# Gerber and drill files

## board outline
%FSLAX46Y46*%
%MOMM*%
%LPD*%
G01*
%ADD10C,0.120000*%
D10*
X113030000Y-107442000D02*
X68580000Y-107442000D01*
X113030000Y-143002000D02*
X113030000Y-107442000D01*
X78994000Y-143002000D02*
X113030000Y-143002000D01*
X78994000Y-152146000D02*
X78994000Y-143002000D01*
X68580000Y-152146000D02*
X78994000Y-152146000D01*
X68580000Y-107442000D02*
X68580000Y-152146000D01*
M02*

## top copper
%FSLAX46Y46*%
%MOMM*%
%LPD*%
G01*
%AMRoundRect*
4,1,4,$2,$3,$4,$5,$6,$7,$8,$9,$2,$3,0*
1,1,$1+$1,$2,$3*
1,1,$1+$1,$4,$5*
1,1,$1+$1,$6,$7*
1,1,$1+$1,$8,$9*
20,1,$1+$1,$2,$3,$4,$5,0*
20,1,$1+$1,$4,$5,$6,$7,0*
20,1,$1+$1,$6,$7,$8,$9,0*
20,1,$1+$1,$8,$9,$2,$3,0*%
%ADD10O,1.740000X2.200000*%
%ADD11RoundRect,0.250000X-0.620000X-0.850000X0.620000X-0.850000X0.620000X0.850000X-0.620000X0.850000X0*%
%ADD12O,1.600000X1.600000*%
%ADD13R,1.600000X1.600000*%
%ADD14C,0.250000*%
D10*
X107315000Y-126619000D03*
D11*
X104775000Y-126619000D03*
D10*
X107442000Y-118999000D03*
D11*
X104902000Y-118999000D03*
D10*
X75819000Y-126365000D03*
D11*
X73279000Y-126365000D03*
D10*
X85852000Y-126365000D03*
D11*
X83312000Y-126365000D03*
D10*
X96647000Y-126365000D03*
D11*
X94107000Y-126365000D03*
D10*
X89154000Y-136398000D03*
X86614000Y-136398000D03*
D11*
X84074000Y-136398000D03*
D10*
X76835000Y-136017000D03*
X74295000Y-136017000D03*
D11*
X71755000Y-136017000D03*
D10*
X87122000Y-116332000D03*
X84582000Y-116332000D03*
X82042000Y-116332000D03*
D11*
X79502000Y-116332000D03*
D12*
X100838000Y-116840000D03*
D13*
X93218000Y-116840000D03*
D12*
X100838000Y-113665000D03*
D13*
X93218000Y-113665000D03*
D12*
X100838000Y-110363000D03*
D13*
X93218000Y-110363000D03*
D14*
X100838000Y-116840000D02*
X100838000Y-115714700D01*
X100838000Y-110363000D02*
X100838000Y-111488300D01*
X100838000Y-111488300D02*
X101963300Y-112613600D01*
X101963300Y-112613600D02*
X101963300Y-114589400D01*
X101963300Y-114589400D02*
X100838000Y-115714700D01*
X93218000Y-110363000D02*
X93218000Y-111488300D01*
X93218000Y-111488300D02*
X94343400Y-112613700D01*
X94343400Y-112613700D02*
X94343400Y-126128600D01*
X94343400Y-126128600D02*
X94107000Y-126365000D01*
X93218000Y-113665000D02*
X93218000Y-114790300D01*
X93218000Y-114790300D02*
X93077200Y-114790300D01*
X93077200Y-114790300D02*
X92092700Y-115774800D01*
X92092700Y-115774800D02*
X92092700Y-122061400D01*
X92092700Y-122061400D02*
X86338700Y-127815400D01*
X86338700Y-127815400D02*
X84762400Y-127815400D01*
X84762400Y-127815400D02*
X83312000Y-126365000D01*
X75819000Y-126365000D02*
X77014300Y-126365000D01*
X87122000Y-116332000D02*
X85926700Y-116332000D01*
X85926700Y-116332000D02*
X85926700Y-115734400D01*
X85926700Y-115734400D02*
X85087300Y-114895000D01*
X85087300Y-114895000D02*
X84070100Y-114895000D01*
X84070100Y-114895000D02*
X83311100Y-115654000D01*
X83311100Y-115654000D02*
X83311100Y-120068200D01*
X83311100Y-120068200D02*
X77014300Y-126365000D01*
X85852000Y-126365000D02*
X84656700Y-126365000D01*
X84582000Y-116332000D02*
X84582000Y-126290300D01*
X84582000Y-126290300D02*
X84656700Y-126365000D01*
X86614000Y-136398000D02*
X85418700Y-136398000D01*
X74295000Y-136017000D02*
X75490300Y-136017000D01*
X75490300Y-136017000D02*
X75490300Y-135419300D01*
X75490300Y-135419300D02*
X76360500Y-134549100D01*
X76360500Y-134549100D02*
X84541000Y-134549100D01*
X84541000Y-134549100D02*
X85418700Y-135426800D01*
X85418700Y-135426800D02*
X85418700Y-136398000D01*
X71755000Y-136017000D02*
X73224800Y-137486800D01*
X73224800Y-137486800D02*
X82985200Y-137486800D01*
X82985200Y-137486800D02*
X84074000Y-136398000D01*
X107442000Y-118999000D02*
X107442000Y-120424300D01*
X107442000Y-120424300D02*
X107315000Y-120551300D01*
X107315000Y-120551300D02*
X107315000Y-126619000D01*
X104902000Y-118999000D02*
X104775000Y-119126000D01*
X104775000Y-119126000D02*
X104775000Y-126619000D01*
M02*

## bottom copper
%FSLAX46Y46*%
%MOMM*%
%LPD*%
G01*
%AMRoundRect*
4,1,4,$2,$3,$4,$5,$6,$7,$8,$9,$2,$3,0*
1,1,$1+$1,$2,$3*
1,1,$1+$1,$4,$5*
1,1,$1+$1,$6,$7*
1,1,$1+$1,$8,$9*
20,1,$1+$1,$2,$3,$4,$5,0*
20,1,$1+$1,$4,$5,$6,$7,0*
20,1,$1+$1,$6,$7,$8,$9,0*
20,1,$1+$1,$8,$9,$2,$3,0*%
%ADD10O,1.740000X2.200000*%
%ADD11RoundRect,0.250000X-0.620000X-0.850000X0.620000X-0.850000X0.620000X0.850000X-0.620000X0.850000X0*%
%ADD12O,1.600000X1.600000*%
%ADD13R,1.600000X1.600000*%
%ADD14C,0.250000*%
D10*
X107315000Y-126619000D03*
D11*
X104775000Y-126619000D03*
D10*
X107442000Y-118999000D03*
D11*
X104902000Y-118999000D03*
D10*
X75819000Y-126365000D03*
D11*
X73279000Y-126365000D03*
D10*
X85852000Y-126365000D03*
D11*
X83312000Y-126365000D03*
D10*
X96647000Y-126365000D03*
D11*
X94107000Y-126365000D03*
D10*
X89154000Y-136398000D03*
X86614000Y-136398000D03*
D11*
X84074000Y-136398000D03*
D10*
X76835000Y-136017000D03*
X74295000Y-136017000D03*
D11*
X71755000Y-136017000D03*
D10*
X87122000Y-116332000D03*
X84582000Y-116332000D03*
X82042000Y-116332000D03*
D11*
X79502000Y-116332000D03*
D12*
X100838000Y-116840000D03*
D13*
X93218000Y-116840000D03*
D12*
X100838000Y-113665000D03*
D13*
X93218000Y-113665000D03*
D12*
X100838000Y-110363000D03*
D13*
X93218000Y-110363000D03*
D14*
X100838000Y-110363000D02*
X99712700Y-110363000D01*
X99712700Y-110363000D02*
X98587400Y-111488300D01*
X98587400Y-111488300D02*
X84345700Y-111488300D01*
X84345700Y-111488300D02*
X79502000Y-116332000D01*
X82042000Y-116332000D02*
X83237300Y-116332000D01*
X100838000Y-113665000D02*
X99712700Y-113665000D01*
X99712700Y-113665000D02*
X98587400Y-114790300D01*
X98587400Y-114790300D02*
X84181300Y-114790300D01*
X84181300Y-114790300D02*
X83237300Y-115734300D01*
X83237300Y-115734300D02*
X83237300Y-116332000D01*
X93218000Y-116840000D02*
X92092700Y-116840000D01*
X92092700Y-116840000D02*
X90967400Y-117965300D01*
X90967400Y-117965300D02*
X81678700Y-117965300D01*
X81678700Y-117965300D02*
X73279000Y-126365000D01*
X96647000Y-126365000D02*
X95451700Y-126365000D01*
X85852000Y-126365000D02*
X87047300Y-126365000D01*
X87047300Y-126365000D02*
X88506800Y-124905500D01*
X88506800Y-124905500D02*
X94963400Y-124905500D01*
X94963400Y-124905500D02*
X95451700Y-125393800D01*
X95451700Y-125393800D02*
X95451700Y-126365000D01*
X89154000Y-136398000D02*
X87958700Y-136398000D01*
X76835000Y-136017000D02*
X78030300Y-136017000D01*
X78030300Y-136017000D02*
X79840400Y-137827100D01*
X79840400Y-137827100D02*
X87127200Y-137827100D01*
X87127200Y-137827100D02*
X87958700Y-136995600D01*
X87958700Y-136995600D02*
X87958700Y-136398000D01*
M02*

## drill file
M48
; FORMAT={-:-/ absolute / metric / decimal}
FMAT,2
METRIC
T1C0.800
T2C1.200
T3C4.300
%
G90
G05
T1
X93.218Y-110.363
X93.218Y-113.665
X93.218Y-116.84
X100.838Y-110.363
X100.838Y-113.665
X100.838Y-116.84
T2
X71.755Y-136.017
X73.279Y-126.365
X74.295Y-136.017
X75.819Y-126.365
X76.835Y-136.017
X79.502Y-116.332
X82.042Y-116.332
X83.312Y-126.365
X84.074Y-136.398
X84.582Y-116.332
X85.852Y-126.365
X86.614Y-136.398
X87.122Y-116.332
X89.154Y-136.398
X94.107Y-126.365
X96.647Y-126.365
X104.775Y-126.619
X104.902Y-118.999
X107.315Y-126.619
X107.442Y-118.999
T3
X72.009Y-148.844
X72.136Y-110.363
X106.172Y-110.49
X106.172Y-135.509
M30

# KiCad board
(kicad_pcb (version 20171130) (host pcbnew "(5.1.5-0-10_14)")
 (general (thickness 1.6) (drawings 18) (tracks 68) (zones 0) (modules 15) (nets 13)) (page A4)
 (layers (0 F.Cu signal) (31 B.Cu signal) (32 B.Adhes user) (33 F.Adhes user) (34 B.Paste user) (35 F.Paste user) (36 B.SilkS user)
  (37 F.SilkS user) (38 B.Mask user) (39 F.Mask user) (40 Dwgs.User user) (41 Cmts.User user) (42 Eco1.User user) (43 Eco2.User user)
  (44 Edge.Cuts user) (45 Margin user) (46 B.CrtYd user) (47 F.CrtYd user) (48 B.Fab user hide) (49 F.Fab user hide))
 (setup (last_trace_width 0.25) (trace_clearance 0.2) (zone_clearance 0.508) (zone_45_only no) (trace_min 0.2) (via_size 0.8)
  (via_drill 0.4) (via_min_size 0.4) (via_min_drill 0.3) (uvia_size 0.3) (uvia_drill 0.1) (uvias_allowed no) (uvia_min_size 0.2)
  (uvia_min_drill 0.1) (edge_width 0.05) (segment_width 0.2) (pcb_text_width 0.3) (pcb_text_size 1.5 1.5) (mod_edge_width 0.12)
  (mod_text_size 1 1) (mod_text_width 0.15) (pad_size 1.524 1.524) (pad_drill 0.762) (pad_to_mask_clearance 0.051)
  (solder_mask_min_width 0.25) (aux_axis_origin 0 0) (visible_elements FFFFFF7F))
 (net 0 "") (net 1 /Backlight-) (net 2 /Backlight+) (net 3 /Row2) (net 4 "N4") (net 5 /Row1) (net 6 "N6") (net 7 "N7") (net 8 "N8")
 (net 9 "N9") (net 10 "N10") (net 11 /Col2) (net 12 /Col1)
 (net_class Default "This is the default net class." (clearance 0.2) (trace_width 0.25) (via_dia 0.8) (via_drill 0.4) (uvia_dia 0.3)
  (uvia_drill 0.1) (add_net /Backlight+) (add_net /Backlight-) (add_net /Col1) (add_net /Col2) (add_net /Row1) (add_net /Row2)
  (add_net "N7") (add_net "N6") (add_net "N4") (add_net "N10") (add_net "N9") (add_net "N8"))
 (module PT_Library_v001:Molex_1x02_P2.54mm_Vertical (layer F.Cu) (at 104.775 126.619)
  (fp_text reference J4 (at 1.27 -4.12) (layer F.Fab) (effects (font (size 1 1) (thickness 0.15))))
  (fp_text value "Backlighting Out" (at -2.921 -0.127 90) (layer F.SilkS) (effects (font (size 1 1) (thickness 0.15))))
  (pad 2 thru_hole oval (at 2.54 0) (size 1.74 2.2) (drill 1.2) (layers *.Cu *.Mask) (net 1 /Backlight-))
  (pad 1 thru_hole roundrect (at 0 0) (size 1.74 2.2) (drill 1.2) (layers *.Cu *.Mask) (roundrect_rratio 0.143678) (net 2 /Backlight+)))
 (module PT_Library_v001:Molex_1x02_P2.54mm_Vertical (layer F.Cu) (at 104.902 118.999)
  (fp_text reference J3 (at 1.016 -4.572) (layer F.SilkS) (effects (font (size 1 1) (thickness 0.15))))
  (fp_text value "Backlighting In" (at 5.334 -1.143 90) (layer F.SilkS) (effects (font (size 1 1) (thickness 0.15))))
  (pad 2 thru_hole oval (at 2.54 0) (size 1.74 2.2) (drill 1.2) (layers *.Cu *.Mask) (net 1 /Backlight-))
  (pad 1 thru_hole roundrect (at 0 0) (size 1.74 2.2) (drill 1.2) (layers *.Cu *.Mask) (roundrect_rratio 0.143678) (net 2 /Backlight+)))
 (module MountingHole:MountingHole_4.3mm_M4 (layer F.Cu) (at 72.009 148.844)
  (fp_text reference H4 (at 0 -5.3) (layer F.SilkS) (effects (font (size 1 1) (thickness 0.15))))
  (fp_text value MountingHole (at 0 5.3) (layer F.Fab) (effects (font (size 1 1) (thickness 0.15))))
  (pad 1 np_thru_hole circle (at 0 0) (size 4.3 4.3) (drill 4.3) (layers *.Cu *.Mask)))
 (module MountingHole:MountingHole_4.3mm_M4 (layer F.Cu) (at 106.172 135.509)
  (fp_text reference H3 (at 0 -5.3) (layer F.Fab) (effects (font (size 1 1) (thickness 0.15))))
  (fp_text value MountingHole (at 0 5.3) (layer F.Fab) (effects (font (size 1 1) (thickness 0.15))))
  (pad 1 np_thru_hole circle (at 0 0) (size 4.3 4.3) (drill 4.3) (layers *.Cu *.Mask)))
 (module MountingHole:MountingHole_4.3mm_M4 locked (layer F.Cu) (at 72.136 110.363)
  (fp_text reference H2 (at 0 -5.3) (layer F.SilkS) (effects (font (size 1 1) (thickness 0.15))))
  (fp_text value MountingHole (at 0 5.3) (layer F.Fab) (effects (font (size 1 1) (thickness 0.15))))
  (pad 1 np_thru_hole circle (at 0 0) (size 4.3 4.3) (drill 4.3) (layers *.Cu *.Mask)))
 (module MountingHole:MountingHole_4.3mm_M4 (layer F.Cu) (at 106.172 110.49)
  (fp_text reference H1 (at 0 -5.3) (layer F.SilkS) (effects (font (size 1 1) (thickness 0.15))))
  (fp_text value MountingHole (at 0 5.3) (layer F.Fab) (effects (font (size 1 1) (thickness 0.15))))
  (pad 1 np_thru_hole circle (at 0 0) (size 4.3 4.3) (drill 4.3) (layers *.Cu *.Mask)))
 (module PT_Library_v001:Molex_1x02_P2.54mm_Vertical (layer F.Cu) (at 73.279 126.365)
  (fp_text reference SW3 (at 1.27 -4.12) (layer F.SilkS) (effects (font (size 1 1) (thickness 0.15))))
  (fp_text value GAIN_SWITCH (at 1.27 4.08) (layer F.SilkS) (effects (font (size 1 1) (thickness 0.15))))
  (pad 2 thru_hole oval (at 2.54 0) (size 1.74 2.2) (drill 1.2) (layers *.Cu *.Mask) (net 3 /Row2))
  (pad 1 thru_hole roundrect (at 0 0) (size 1.74 2.2) (drill 1.2) (layers *.Cu *.Mask) (roundrect_rratio 0.143678) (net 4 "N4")))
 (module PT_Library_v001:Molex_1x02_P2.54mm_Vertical (layer F.Cu) (at 83.312 126.365)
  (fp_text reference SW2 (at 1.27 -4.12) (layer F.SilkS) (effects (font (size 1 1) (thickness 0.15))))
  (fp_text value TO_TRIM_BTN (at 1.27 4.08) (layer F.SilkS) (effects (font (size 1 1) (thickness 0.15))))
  (pad 2 thru_hole oval (at 2.54 0) (size 1.74 2.2) (drill 1.2) (layers *.Cu *.Mask) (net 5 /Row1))
  (pad 1 thru_hole roundrect (at 0 0) (size 1.74 2.2) (drill 1.2) (layers *.Cu *.Mask) (roundrect_rratio 0.143678) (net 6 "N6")))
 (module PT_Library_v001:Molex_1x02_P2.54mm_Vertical (layer F.Cu) (at 94.107 126.365)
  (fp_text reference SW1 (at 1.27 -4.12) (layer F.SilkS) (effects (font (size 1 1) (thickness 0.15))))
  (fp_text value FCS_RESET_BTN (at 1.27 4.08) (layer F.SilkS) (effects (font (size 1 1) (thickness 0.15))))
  (pad 2 thru_hole oval (at 2.54 0) (size 1.74 2.2) (drill 1.2) (layers *.Cu *.Mask) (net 5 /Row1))
  (pad 1 thru_hole roundrect (at 0 0) (size 1.74 2.2) (drill 1.2) (layers *.Cu *.Mask) (roundrect_rratio 0.143678) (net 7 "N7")))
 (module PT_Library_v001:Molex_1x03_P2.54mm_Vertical (layer F.Cu) (at 84.074 136.398)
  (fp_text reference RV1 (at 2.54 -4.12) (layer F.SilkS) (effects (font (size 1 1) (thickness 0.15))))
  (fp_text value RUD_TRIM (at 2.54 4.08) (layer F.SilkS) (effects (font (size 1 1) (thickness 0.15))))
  (pad 3 thru_hole oval (at 5.08 0) (size 1.74 2.2) (drill 1.2) (layers *.Cu *.Mask) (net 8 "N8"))
  (pad 2 thru_hole oval (at 2.54 0) (size 1.74 2.2) (drill 1.2) (layers *.Cu *.Mask) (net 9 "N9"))
  (pad 1 thru_hole roundrect (at 0 0) (size 1.74 2.2) (drill 1.2) (layers *.Cu *.Mask) (roundrect_rratio 0.143678) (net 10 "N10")))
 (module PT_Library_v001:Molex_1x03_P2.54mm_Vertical (layer F.Cu) (at 71.755 136.017)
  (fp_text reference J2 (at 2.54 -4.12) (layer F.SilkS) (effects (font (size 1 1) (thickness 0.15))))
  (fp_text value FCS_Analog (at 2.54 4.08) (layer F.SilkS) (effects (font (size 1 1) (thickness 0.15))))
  (pad 3 thru_hole oval (at 5.08 0) (size 1.74 2.2) (drill 1.2) (layers *.Cu *.Mask) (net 8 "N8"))
  (pad 2 thru_hole oval (at 2.54 0) (size 1.74 2.2) (drill 1.2) (layers *.Cu *.Mask) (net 9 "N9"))
  (pad 1 thru_hole roundrect (at 0 0) (size 1.74 2.2) (drill 1.2) (layers *.Cu *.Mask) (roundrect_rratio 0.143678) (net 10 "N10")))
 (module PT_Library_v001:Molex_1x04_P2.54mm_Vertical (layer F.Cu) (at 79.502 116.332)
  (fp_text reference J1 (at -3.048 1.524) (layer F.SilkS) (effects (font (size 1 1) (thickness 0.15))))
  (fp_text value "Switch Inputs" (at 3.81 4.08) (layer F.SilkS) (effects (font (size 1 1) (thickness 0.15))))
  (pad 4 thru_hole oval (at 7.62 0) (size 1.74 2.2) (drill 1.2) (layers *.Cu *.Mask) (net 3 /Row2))
  (pad 3 thru_hole oval (at 5.08 0) (size 1.74 2.2) (drill 1.2) (layers *.Cu *.Mask) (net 5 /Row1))
  (pad 2 thru_hole oval (at 2.54 0) (size 1.74 2.2) (drill 1.2) (layers *.Cu *.Mask) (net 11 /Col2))
  (pad 1 thru_hole roundrect (at 0 0) (size 1.74 2.2) (drill 1.2) (layers *.Cu *.Mask) (roundrect_rratio 0.143678) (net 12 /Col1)))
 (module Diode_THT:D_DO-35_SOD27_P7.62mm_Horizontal (layer F.Cu) (at 93.218 116.84)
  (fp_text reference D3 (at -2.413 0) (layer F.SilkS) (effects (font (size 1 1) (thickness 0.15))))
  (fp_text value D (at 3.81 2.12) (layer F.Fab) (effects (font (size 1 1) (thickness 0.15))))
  (pad 2 thru_hole oval (at 7.62 0) (size 1.6 1.6) (drill 0.8) (layers *.Cu *.Mask) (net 12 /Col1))
  (pad 1 thru_hole rect (at 0 0) (size 1.6 1.6) (drill 0.8) (layers *.Cu *.Mask) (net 4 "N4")))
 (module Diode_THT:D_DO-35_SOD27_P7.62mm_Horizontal (layer F.Cu) (at 93.218 113.665)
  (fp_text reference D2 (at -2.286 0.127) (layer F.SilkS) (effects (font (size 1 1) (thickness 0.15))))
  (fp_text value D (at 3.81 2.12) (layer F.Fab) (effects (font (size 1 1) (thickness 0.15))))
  (pad 2 thru_hole oval (at 7.62 0) (size 1.6 1.6) (drill 0.8) (layers *.Cu *.Mask) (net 11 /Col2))
  (pad 1 thru_hole rect (at 0 0) (size 1.6 1.6) (drill 0.8) (layers *.Cu *.Mask) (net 6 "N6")))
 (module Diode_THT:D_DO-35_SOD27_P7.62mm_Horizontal (layer F.Cu) (at 93.218 110.363)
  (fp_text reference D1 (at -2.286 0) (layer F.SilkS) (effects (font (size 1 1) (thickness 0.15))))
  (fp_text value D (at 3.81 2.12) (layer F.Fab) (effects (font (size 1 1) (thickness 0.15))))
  (pad 2 thru_hole oval (at 7.62 0) (size 1.6 1.6) (drill 0.8) (layers *.Cu *.Mask) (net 12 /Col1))
  (pad 1 thru_hole rect (at 0 0) (size 1.6 1.6) (drill 0.8) (layers *.Cu *.Mask) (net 7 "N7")))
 (gr_line (start 113.03 107.442) (end 68.58 107.442) (layer Edge.Cuts) (width 0.12))
 (gr_line (start 113.03 143.002) (end 113.03 107.442) (layer Edge.Cuts) (width 0.12))
 (gr_line (start 78.994 143.002) (end 113.03 143.002) (layer Edge.Cuts) (width 0.12))
 (gr_line (start 78.994 152.146) (end 78.994 143.002) (layer Edge.Cuts) (width 0.12))
 (gr_line (start 68.58 152.146) (end 78.994 152.146) (layer Edge.Cuts) (width 0.12))
 (gr_line (start 68.58 107.442) (end 68.58 152.146) (layer Edge.Cuts) (width 0.12))
 (segment (start 100.838 116.84) (end 100.838 115.7147) (width 0.25) (layer F.Cu) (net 12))
 (segment (start 100.838 110.363) (end 100.838 111.4883) (width 0.25) (layer F.Cu) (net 12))
 (segment (start 100.838 111.4883) (end 101.9633 112.6136) (width 0.25) (layer F.Cu) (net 12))
 (segment (start 101.9633 112.6136) (end 101.9633 114.5894) (width 0.25) (layer F.Cu) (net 12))
 (segment (start 101.9633 114.5894) (end 100.838 115.7147) (width 0.25) (layer F.Cu) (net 12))
 (segment (start 100.838 110.363) (end 99.7127 110.363) (width 0.25) (layer B.Cu) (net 12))
 (segment (start 99.7127 110.363) (end 98.5874 111.4883) (width 0.25) (layer B.Cu) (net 12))
 (segment (start 98.5874 111.4883) (end 84.3457 111.4883) (width 0.25) (layer B.Cu) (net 12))
 (segment (start 84.3457 111.4883) (end 79.502 116.332) (width 0.25) (layer B.Cu) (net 12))
 (segment (start 93.218 110.363) (end 93.218 111.4883) (width 0.25) (layer F.Cu) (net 7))
 (segment (start 93.218 111.4883) (end 94.3434 112.6137) (width 0.25) (layer F.Cu) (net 7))
 (segment (start 94.3434 112.6137) (end 94.3434 126.1286) (width 0.25) (layer F.Cu) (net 7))
 (segment (start 94.3434 126.1286) (end 94.107 126.365) (width 0.25) (layer F.Cu) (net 7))
 (segment (start 82.042 116.332) (end 83.2373 116.332) (width 0.25) (layer B.Cu) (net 11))
 (segment (start 100.838 113.665) (end 99.7127 113.665) (width 0.25) (layer B.Cu) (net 11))
 (segment (start 99.7127 113.665) (end 98.5874 114.7903) (width 0.25) (layer B.Cu) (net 11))
 (segment (start 98.5874 114.7903) (end 84.1813 114.7903) (width 0.25) (layer B.Cu) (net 11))
 (segment (start 84.1813 114.7903) (end 83.2373 115.7343) (width 0.25) (layer B.Cu) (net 11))
 (segment (start 83.2373 115.7343) (end 83.2373 116.332) (width 0.25) (layer B.Cu) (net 11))
 (segment (start 93.218 113.665) (end 93.218 114.7903) (width 0.25) (layer F.Cu) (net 6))
 (segment (start 93.218 114.7903) (end 93.0772 114.7903) (width 0.25) (layer F.Cu) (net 6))
 (segment (start 93.0772 114.7903) (end 92.0927 115.7748) (width 0.25) (layer F.Cu) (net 6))
 (segment (start 92.0927 115.7748) (end 92.0927 122.0614) (width 0.25) (layer F.Cu) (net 6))
 (segment (start 92.0927 122.0614) (end 86.3387 127.8154) (width 0.25) (layer F.Cu) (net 6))
 (segment (start 86.3387 127.8154) (end 84.7624 127.8154) (width 0.25) (layer F.Cu) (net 6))
 (segment (start 84.7624 127.8154) (end 83.312 126.365) (width 0.25) (layer F.Cu) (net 6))
 (segment (start 93.218 116.84) (end 92.0927 116.84) (width 0.25) (layer B.Cu) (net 4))
 (segment (start 92.0927 116.84) (end 90.9674 117.9653) (width 0.25) (layer B.Cu) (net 4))
 (segment (start 90.9674 117.9653) (end 81.6787 117.9653) (width 0.25) (layer B.Cu) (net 4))
 (segment (start 81.6787 117.9653) (end 73.279 126.365) (width 0.25) (layer B.Cu) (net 4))
 (segment (start 75.819 126.365) (end 77.0143 126.365) (width 0.25) (layer F.Cu) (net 3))
 (segment (start 87.122 116.332) (end 85.9267 116.332) (width 0.25) (layer F.Cu) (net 3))
 (segment (start 85.9267 116.332) (end 85.9267 115.7344) (width 0.25) (layer F.Cu) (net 3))
 (segment (start 85.9267 115.7344) (end 85.0873 114.895) (width 0.25) (layer F.Cu) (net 3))
 (segment (start 85.0873 114.895) (end 84.0701 114.895) (width 0.25) (layer F.Cu) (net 3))
 (segment (start 84.0701 114.895) (end 83.3111 115.654) (width 0.25) (layer F.Cu) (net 3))
 (segment (start 83.3111 115.654) (end 83.3111 120.0682) (width 0.25) (layer F.Cu) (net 3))
 (segment (start 83.3111 120.0682) (end 77.0143 126.365) (width 0.25) (layer F.Cu) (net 3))
 (segment (start 85.852 126.365) (end 84.6567 126.365) (width 0.25) (layer F.Cu) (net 5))
 (segment (start 84.582 116.332) (end 84.582 126.2903) (width 0.25) (layer F.Cu) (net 5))
 (segment (start 84.582 126.2903) (end 84.6567 126.365) (width 0.25) (layer F.Cu) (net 5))
 (segment (start 96.647 126.365) (end 95.4517 126.365) (width 0.25) (layer B.Cu) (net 5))
 (segment (start 85.852 126.365) (end 87.0473 126.365) (width 0.25) (layer B.Cu) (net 5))
 (segment (start 87.0473 126.365) (end 88.5068 124.9055) (width 0.25) (layer B.Cu) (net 5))
 (segment (start 88.5068 124.9055) (end 94.9634 124.9055) (width 0.25) (layer B.Cu) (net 5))
 (segment (start 94.9634 124.9055) (end 95.4517 125.3938) (width 0.25) (layer B.Cu) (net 5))
 (segment (start 95.4517 125.3938) (end 95.4517 126.365) (width 0.25) (layer B.Cu) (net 5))
 (segment (start 89.154 136.398) (end 87.9587 136.398) (width 0.25) (layer B.Cu) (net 8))
 (segment (start 76.835 136.017) (end 78.0303 136.017) (width 0.25) (layer B.Cu) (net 8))
 (segment (start 78.0303 136.017) (end 79.8404 137.8271) (width 0.25) (layer B.Cu) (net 8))
 (segment (start 79.8404 137.8271) (end 87.1272 137.8271) (width 0.25) (layer B.Cu) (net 8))
 (segment (start 87.1272 137.8271) (end 87.9587 136.9956) (width 0.25) (layer B.Cu) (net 8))
 (segment (start 87.9587 136.9956) (end 87.9587 136.398) (width 0.25) (layer B.Cu) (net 8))
 (segment (start 86.614 136.398) (end 85.4187 136.398) (width 0.25) (layer F.Cu) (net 9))
 (segment (start 74.295 136.017) (end 75.4903 136.017) (width 0.25) (layer F.Cu) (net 9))
 (segment (start 75.4903 136.017) (end 75.4903 135.4193) (width 0.25) (layer F.Cu) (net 9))
 (segment (start 75.4903 135.4193) (end 76.3605 134.5491) (width 0.25) (layer F.Cu) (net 9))
 (segment (start 76.3605 134.5491) (end 84.541 134.5491) (width 0.25) (layer F.Cu) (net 9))
 (segment (start 84.541 134.5491) (end 85.4187 135.4268) (width 0.25) (layer F.Cu) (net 9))
 (segment (start 85.4187 135.4268) (end 85.4187 136.398) (width 0.25) (layer F.Cu) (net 9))
 (segment (start 71.755 136.017) (end 73.2248 137.4868) (width 0.25) (layer F.Cu) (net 10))
 (segment (start 73.2248 137.4868) (end 82.9852 137.4868) (width 0.25) (layer F.Cu) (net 10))
 (segment (start 82.9852 137.4868) (end 84.074 136.398) (width 0.25) (layer F.Cu) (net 10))
 (segment (start 107.442 118.999) (end 107.442 120.4243) (width 0.25) (layer F.Cu) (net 1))
 (segment (start 107.442 120.4243) (end 107.315 120.5513) (width 0.25) (layer F.Cu) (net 1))
 (segment (start 107.315 120.5513) (end 107.315 126.619) (width 0.25) (layer F.Cu) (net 1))
 (segment (start 104.902 118.999) (end 104.775 119.126) (width 0.25) (layer F.Cu) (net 2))
 (segment (start 104.775 119.126) (end 104.775 126.619) (width 0.25) (layer F.Cu) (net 2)))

